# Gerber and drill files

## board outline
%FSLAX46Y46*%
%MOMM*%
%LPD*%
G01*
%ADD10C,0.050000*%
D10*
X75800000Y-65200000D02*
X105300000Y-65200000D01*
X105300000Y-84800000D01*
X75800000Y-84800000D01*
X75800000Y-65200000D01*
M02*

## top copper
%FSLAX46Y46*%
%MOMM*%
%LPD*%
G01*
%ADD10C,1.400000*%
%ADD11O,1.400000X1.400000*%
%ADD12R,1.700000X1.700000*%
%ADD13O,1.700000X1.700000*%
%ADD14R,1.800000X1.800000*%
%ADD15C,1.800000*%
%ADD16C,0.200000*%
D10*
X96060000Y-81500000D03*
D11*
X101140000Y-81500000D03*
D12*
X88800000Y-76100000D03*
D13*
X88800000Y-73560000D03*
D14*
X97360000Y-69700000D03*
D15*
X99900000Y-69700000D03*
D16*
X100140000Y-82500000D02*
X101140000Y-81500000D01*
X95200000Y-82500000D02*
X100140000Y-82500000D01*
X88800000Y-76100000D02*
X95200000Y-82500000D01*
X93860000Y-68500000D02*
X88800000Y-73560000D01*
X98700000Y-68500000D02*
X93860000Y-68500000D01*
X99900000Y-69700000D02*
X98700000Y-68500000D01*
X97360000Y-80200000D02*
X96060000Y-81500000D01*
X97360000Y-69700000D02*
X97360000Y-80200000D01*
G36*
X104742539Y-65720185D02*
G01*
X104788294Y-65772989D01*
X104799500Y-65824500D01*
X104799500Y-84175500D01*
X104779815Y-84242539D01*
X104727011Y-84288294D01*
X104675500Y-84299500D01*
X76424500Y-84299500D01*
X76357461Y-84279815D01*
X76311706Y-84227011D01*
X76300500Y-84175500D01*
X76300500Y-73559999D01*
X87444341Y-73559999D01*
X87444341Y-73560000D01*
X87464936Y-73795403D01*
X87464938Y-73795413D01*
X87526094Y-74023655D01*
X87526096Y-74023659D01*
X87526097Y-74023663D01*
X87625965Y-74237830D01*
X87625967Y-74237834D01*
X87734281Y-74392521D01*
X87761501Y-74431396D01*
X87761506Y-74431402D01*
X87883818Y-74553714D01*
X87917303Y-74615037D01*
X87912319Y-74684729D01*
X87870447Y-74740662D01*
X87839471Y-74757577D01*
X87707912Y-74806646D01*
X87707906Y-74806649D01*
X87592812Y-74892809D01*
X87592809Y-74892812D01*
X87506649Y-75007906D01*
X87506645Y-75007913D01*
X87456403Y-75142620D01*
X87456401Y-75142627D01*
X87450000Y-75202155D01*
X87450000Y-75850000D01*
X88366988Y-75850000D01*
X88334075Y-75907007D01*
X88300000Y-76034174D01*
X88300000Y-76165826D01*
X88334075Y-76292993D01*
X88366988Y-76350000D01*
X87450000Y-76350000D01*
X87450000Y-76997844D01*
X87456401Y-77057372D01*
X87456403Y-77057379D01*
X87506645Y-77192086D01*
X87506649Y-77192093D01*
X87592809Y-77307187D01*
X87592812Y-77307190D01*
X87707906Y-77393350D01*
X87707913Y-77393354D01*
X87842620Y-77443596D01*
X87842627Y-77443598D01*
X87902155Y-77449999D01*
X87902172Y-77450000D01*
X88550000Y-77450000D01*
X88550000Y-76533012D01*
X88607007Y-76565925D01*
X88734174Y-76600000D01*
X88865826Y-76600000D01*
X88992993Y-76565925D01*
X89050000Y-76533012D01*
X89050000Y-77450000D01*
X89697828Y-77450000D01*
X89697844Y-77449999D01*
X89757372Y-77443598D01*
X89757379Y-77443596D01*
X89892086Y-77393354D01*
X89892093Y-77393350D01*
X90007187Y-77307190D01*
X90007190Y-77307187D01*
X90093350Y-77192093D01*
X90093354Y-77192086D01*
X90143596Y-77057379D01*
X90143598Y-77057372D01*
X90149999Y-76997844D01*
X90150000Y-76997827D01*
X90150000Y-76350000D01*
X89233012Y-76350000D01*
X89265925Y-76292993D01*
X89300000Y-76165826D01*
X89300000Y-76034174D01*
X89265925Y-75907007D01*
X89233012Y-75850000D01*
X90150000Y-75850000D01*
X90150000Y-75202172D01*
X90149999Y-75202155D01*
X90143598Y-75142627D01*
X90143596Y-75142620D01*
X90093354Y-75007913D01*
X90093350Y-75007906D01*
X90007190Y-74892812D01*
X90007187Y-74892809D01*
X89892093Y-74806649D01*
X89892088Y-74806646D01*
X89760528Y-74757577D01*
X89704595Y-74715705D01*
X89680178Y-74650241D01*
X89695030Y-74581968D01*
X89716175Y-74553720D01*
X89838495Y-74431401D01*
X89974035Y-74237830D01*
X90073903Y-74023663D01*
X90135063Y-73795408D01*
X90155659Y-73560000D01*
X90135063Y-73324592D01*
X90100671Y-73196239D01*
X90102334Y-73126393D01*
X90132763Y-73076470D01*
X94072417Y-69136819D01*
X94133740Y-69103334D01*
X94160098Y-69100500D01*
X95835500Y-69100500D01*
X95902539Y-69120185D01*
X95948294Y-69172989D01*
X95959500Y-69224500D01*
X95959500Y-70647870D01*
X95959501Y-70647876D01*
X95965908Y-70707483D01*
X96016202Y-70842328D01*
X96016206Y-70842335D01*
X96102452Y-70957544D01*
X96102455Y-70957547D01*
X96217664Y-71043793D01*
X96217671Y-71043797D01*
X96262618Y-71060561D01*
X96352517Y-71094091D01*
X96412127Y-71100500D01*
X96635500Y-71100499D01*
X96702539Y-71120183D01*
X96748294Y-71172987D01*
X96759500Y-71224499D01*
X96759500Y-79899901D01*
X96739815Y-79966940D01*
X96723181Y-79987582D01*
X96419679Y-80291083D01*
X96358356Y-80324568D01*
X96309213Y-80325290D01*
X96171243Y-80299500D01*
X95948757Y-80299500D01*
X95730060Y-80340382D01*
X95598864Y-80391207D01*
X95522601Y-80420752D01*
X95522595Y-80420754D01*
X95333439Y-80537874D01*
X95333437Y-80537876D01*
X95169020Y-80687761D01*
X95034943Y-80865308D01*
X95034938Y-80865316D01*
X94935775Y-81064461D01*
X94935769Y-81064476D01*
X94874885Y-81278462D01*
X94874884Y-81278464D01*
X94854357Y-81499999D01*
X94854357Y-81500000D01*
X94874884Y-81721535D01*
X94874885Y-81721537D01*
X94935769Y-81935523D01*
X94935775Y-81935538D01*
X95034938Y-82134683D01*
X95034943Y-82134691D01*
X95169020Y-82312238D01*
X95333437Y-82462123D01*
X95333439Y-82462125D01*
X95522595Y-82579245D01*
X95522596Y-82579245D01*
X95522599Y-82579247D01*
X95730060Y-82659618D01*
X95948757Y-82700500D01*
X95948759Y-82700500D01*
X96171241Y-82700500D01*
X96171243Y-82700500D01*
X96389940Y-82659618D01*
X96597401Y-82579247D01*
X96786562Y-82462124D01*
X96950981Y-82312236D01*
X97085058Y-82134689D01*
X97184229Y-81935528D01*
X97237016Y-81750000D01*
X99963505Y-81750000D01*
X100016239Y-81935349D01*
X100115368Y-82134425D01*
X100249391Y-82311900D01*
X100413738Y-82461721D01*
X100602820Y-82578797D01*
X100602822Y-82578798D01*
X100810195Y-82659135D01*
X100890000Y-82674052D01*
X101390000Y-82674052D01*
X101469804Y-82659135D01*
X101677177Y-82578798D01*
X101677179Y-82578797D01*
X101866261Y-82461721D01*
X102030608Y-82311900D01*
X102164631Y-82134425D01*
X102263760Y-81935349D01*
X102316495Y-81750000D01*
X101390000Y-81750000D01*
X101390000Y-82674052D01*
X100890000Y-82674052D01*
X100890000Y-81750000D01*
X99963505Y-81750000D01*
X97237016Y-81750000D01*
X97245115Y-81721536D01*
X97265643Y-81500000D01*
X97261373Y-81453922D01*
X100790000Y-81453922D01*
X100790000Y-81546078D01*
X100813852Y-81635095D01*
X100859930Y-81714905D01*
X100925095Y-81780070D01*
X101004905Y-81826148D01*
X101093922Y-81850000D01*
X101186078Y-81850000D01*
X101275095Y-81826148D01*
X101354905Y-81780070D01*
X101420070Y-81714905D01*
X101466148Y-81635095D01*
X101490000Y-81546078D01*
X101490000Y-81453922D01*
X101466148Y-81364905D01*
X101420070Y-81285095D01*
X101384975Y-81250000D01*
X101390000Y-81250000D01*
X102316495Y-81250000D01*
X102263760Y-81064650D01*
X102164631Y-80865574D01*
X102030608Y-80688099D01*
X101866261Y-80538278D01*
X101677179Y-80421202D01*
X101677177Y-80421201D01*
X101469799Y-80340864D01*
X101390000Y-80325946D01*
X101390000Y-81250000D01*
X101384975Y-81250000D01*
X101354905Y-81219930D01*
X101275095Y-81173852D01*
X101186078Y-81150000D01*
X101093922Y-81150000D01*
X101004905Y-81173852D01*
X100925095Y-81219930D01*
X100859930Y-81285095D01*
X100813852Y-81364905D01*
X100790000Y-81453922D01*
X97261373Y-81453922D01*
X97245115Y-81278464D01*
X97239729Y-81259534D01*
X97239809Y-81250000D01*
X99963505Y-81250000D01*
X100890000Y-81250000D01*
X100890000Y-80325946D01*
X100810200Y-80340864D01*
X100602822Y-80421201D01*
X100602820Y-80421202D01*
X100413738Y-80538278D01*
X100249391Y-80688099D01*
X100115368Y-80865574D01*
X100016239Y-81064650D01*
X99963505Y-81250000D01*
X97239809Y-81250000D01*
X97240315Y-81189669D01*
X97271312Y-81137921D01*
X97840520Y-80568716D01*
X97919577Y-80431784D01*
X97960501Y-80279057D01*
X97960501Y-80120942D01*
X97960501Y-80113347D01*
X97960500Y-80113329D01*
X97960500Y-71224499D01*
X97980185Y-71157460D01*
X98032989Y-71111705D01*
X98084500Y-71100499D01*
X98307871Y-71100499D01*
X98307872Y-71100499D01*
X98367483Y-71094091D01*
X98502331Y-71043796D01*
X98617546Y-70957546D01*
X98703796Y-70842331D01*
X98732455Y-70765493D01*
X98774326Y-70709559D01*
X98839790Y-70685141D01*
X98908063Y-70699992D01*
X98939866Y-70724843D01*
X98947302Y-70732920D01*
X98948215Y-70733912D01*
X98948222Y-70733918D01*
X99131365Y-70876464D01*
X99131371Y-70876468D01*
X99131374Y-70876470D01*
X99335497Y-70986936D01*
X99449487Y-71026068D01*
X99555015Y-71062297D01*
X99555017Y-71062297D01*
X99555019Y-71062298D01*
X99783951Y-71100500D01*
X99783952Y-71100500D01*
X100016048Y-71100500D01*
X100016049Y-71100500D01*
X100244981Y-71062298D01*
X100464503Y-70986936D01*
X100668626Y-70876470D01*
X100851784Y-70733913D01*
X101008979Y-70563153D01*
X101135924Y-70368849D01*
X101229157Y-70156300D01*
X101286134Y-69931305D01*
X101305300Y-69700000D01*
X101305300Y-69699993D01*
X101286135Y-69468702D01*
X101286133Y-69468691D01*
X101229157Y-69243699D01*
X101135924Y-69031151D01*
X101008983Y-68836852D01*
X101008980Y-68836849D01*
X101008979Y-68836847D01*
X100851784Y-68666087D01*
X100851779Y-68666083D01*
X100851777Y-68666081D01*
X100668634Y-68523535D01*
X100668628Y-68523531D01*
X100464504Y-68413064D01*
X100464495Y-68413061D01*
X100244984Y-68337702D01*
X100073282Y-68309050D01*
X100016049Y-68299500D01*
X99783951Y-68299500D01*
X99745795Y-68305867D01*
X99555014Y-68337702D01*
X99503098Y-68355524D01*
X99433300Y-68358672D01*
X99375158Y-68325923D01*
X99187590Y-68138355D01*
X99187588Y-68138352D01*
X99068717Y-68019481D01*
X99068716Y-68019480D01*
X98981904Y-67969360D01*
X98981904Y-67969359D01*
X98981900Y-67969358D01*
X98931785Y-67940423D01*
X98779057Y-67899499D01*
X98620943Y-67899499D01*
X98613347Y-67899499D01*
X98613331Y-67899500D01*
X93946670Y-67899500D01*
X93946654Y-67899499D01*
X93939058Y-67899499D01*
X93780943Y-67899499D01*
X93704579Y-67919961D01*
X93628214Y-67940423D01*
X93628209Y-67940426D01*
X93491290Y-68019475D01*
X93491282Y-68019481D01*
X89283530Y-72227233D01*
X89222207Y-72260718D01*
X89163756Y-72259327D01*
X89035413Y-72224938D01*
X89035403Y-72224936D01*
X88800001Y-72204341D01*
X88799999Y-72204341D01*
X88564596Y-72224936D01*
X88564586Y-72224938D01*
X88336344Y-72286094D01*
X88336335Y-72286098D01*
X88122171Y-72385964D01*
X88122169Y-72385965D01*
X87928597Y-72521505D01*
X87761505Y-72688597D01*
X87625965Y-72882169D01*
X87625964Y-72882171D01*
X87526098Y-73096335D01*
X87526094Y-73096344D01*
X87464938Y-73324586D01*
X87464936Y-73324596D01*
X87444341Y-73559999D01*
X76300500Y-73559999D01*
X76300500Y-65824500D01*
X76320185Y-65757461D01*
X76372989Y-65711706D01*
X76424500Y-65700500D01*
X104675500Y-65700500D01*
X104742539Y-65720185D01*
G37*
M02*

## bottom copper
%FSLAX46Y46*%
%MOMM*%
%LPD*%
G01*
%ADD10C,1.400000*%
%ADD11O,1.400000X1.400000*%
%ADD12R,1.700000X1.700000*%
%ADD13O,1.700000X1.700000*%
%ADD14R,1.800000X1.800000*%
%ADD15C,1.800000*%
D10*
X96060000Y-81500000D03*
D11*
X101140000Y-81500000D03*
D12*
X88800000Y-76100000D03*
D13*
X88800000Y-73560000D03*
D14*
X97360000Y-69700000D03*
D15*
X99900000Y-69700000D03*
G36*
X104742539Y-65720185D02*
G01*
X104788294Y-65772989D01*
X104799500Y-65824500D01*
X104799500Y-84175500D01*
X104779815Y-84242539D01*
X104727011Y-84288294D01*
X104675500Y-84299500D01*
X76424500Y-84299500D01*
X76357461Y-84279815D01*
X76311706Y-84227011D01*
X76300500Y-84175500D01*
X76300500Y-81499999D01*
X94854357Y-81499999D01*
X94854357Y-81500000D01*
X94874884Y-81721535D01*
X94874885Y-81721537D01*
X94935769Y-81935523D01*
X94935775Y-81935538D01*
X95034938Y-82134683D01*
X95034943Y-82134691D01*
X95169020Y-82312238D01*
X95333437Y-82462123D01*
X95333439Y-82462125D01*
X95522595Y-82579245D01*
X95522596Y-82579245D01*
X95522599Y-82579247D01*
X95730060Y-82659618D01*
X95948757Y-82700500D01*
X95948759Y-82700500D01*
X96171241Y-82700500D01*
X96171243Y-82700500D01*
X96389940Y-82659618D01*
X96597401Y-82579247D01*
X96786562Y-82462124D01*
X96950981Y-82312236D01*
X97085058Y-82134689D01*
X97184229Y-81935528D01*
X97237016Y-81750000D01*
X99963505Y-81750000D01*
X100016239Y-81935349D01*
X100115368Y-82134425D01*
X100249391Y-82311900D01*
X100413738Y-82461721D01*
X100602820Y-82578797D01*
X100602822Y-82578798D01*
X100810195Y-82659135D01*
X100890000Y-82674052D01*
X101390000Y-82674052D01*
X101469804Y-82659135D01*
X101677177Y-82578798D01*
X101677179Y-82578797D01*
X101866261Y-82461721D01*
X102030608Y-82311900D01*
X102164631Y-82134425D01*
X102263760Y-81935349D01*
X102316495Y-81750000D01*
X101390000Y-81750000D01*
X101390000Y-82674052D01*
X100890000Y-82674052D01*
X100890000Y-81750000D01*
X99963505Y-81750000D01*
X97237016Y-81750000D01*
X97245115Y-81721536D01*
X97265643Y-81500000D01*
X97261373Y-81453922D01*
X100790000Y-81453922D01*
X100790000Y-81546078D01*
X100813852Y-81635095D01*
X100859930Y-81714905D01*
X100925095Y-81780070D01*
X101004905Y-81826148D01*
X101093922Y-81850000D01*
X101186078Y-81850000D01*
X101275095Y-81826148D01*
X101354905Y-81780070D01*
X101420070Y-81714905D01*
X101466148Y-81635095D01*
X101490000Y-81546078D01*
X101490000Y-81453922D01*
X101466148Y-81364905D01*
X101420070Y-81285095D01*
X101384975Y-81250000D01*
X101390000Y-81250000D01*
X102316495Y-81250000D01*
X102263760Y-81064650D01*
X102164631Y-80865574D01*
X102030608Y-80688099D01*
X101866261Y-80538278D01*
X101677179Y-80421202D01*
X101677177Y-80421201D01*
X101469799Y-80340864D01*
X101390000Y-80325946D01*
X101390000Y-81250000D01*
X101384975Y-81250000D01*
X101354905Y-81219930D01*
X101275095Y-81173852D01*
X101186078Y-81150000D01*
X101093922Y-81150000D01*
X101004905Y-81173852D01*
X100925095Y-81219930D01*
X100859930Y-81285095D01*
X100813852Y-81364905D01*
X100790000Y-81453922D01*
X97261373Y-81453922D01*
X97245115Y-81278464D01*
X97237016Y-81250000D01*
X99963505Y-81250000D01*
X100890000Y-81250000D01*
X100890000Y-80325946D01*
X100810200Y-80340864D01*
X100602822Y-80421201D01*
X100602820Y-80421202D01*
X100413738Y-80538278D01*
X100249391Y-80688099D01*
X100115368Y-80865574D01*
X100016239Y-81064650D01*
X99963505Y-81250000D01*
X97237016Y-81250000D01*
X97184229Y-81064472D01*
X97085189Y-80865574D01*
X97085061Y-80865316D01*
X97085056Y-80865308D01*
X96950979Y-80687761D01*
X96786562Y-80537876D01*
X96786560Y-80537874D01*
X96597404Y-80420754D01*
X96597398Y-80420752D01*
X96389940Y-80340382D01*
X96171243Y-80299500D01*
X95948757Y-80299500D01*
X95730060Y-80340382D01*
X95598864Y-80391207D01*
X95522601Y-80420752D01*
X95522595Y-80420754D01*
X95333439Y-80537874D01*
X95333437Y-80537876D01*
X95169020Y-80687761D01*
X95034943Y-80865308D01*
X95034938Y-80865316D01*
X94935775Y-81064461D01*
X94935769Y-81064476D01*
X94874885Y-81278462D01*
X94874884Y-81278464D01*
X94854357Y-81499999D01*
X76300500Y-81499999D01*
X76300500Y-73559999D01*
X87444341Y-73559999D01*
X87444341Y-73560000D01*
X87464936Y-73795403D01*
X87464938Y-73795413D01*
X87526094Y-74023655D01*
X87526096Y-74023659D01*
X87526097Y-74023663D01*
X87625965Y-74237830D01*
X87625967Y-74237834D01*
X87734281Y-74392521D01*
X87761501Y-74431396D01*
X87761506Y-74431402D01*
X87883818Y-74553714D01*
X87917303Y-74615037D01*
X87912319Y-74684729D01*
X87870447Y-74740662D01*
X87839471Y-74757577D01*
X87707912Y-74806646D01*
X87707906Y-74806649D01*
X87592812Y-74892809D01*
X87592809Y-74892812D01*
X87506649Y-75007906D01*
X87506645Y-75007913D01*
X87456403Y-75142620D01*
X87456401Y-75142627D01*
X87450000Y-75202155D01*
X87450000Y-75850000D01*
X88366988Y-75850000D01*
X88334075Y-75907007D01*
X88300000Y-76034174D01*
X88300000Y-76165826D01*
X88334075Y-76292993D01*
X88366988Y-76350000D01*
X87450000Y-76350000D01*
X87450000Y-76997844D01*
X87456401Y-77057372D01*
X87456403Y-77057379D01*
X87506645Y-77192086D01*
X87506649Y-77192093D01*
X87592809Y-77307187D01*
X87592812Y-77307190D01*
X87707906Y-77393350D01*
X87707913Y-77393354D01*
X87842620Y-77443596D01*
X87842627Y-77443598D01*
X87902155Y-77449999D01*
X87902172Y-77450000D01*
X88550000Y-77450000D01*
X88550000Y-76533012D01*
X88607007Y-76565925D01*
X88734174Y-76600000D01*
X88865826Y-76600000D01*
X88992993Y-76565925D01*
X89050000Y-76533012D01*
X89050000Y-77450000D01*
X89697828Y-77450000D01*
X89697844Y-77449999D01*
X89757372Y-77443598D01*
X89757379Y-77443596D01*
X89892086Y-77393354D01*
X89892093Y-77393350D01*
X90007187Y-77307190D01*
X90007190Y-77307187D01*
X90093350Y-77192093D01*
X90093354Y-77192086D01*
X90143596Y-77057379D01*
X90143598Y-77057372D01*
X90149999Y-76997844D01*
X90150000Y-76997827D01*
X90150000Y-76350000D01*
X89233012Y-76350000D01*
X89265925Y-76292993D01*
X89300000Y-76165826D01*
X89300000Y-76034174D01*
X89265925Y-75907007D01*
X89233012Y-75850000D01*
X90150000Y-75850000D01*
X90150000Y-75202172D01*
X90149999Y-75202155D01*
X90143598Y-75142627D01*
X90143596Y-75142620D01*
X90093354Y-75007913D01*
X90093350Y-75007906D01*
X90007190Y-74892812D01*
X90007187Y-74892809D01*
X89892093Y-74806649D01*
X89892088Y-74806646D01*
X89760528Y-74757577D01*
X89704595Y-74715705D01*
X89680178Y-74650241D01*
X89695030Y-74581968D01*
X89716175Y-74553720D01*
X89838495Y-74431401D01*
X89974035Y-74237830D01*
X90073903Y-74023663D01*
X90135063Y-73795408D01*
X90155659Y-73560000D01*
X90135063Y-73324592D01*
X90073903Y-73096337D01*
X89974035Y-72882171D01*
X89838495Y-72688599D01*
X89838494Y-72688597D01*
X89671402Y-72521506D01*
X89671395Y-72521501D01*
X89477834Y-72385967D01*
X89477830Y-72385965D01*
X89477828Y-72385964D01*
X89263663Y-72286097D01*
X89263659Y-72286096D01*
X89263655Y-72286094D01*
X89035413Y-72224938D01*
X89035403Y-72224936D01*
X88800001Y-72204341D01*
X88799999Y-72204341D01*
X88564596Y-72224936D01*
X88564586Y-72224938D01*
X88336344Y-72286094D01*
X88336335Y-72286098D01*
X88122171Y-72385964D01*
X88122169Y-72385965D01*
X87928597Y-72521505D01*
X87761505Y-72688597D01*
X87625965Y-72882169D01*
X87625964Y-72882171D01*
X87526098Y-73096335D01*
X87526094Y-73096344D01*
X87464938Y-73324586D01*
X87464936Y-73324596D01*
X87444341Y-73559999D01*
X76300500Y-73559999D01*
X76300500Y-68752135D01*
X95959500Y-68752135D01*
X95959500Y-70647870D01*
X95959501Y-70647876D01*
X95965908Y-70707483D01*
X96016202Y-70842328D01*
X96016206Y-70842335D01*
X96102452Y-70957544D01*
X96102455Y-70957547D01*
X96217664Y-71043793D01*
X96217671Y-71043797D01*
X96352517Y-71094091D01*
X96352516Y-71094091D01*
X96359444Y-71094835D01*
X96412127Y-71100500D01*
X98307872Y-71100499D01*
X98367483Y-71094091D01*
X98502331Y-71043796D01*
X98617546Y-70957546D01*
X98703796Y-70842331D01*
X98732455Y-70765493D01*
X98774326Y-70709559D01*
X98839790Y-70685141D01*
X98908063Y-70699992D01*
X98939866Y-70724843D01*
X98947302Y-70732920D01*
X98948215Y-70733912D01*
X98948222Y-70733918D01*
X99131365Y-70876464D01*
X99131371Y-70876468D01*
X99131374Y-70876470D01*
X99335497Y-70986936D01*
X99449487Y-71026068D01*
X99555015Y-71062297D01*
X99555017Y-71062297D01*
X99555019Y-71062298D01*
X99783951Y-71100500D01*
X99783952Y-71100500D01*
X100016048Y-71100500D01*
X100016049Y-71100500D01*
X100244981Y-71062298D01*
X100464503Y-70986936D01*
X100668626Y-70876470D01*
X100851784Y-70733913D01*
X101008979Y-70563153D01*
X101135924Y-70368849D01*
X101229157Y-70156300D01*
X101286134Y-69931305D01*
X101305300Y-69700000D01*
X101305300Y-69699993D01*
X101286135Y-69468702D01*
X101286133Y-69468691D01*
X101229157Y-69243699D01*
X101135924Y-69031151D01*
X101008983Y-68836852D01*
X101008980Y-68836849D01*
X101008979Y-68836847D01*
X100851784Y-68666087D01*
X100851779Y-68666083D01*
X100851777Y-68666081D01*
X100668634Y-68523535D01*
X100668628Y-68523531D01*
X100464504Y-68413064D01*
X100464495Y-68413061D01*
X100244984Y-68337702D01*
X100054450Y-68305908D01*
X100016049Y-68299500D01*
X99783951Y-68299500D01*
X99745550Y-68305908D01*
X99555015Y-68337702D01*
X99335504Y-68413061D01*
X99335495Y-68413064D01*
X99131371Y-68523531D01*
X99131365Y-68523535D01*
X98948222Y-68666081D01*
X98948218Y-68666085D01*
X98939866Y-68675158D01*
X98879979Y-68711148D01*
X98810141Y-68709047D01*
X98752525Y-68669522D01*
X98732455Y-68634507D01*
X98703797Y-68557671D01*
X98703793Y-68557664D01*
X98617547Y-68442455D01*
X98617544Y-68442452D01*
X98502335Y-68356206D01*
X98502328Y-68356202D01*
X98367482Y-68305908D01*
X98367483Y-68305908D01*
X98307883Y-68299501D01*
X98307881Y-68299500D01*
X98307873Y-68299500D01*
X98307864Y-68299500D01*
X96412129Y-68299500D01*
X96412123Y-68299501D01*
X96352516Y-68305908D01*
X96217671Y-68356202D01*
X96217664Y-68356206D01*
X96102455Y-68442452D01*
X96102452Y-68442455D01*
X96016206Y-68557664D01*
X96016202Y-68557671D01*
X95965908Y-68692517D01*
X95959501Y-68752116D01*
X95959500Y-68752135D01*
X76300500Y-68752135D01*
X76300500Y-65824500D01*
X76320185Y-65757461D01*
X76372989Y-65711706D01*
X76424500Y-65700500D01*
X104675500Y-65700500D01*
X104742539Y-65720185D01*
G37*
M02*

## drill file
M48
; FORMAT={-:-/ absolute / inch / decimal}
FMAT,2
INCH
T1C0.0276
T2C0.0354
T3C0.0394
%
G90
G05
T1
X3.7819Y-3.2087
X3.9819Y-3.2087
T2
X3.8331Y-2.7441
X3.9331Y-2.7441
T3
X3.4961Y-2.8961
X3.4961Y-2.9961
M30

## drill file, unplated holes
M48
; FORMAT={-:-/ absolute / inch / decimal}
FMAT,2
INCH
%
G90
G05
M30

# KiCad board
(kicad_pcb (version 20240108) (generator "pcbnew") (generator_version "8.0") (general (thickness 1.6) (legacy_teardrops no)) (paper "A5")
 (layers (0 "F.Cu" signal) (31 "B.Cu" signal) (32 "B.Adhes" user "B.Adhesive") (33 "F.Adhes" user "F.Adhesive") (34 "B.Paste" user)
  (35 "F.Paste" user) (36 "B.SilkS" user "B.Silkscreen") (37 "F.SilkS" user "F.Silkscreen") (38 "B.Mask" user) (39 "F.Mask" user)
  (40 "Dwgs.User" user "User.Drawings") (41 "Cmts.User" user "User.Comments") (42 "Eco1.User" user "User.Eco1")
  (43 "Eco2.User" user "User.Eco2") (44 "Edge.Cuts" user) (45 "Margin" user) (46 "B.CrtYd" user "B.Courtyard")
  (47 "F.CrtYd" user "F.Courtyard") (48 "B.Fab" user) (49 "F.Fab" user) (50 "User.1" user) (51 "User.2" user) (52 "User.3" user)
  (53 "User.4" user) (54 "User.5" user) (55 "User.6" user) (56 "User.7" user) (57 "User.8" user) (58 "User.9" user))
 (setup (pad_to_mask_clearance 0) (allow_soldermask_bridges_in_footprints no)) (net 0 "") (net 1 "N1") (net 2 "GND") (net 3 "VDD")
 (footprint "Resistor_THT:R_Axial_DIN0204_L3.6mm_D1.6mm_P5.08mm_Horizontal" (layer "F.Cu") (at 96.06 81.5)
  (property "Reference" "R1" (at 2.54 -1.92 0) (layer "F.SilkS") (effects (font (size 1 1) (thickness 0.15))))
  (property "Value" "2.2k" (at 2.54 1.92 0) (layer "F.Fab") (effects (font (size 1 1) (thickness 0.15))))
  (pad "1" thru_hole circle (at 0 0) (size 1.4 1.4) (drill 0.7) (layers "*.Cu" "*.Mask") (remove_unused_layers no) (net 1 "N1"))
  (pad "2" thru_hole oval (at 5.08 0) (size 1.4 1.4) (drill 0.7) (layers "*.Cu" "*.Mask") (remove_unused_layers no) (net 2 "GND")))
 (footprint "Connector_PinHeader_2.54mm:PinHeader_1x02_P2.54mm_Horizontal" (layer "F.Cu") (at 88.8 76.1 180)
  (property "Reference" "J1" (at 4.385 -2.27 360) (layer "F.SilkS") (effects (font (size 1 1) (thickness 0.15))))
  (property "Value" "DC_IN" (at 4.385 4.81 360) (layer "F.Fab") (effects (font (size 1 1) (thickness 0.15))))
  (pad "1" thru_hole rect (at 0 0 180) (size 1.7 1.7) (drill 1) (layers "*.Cu" "*.Mask") (remove_unused_layers no) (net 2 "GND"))
  (pad "2" thru_hole oval (at 0 2.54 180) (size 1.7 1.7) (drill 1) (layers "*.Cu" "*.Mask") (remove_unused_layers no) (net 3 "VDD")))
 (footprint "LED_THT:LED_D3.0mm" (layer "F.Cu") (at 97.36 69.7)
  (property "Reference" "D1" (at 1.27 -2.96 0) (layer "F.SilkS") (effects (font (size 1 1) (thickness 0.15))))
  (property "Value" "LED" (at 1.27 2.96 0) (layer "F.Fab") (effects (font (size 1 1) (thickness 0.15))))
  (pad "1" thru_hole rect (at 0 0) (size 1.8 1.8) (drill 0.9) (layers "*.Cu" "*.Mask") (remove_unused_layers no) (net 1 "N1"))
  (pad "2" thru_hole circle (at 2.54 0) (size 1.8 1.8) (drill 0.9) (layers "*.Cu" "*.Mask") (remove_unused_layers no) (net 3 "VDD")))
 (gr_rect (start 75.8 65.2) (end 105.3 84.8) (stroke (width 0.05) (type default)) (fill none) (layer "Edge.Cuts"))
 (segment (start 93.86 68.5) (end 88.8 73.56) (width 0.2) (layer "F.Cu") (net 3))
 (segment (start 98.7 68.5) (end 93.86 68.5) (width 0.2) (layer "F.Cu") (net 3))
 (segment (start 99.9 69.7) (end 98.7 68.5) (width 0.2) (layer "F.Cu") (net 3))
 (segment (start 97.36 80.2) (end 96.06 81.5) (width 0.2) (layer "F.Cu") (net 1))
 (segment (start 97.36 69.7) (end 97.36 80.2) (width 0.2) (layer "F.Cu") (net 1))
 (segment (start 100.14 82.5) (end 101.14 81.5) (width 0.2) (layer "F.Cu") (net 2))
 (segment (start 88.8 76.1) (end 95.2 82.5) (width 0.2) (layer "F.Cu") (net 2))
 (segment (start 95.2 82.5) (end 100.14 82.5) (width 0.2) (layer "F.Cu") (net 2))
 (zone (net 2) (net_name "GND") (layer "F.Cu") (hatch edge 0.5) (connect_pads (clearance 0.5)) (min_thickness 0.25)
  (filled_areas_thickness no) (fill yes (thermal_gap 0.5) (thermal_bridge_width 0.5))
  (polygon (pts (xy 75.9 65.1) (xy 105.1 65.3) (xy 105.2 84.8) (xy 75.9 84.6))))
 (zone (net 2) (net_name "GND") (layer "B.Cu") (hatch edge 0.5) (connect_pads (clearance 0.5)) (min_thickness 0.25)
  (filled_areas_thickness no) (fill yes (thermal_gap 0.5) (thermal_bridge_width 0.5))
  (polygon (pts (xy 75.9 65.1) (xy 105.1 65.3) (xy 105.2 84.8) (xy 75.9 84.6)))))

